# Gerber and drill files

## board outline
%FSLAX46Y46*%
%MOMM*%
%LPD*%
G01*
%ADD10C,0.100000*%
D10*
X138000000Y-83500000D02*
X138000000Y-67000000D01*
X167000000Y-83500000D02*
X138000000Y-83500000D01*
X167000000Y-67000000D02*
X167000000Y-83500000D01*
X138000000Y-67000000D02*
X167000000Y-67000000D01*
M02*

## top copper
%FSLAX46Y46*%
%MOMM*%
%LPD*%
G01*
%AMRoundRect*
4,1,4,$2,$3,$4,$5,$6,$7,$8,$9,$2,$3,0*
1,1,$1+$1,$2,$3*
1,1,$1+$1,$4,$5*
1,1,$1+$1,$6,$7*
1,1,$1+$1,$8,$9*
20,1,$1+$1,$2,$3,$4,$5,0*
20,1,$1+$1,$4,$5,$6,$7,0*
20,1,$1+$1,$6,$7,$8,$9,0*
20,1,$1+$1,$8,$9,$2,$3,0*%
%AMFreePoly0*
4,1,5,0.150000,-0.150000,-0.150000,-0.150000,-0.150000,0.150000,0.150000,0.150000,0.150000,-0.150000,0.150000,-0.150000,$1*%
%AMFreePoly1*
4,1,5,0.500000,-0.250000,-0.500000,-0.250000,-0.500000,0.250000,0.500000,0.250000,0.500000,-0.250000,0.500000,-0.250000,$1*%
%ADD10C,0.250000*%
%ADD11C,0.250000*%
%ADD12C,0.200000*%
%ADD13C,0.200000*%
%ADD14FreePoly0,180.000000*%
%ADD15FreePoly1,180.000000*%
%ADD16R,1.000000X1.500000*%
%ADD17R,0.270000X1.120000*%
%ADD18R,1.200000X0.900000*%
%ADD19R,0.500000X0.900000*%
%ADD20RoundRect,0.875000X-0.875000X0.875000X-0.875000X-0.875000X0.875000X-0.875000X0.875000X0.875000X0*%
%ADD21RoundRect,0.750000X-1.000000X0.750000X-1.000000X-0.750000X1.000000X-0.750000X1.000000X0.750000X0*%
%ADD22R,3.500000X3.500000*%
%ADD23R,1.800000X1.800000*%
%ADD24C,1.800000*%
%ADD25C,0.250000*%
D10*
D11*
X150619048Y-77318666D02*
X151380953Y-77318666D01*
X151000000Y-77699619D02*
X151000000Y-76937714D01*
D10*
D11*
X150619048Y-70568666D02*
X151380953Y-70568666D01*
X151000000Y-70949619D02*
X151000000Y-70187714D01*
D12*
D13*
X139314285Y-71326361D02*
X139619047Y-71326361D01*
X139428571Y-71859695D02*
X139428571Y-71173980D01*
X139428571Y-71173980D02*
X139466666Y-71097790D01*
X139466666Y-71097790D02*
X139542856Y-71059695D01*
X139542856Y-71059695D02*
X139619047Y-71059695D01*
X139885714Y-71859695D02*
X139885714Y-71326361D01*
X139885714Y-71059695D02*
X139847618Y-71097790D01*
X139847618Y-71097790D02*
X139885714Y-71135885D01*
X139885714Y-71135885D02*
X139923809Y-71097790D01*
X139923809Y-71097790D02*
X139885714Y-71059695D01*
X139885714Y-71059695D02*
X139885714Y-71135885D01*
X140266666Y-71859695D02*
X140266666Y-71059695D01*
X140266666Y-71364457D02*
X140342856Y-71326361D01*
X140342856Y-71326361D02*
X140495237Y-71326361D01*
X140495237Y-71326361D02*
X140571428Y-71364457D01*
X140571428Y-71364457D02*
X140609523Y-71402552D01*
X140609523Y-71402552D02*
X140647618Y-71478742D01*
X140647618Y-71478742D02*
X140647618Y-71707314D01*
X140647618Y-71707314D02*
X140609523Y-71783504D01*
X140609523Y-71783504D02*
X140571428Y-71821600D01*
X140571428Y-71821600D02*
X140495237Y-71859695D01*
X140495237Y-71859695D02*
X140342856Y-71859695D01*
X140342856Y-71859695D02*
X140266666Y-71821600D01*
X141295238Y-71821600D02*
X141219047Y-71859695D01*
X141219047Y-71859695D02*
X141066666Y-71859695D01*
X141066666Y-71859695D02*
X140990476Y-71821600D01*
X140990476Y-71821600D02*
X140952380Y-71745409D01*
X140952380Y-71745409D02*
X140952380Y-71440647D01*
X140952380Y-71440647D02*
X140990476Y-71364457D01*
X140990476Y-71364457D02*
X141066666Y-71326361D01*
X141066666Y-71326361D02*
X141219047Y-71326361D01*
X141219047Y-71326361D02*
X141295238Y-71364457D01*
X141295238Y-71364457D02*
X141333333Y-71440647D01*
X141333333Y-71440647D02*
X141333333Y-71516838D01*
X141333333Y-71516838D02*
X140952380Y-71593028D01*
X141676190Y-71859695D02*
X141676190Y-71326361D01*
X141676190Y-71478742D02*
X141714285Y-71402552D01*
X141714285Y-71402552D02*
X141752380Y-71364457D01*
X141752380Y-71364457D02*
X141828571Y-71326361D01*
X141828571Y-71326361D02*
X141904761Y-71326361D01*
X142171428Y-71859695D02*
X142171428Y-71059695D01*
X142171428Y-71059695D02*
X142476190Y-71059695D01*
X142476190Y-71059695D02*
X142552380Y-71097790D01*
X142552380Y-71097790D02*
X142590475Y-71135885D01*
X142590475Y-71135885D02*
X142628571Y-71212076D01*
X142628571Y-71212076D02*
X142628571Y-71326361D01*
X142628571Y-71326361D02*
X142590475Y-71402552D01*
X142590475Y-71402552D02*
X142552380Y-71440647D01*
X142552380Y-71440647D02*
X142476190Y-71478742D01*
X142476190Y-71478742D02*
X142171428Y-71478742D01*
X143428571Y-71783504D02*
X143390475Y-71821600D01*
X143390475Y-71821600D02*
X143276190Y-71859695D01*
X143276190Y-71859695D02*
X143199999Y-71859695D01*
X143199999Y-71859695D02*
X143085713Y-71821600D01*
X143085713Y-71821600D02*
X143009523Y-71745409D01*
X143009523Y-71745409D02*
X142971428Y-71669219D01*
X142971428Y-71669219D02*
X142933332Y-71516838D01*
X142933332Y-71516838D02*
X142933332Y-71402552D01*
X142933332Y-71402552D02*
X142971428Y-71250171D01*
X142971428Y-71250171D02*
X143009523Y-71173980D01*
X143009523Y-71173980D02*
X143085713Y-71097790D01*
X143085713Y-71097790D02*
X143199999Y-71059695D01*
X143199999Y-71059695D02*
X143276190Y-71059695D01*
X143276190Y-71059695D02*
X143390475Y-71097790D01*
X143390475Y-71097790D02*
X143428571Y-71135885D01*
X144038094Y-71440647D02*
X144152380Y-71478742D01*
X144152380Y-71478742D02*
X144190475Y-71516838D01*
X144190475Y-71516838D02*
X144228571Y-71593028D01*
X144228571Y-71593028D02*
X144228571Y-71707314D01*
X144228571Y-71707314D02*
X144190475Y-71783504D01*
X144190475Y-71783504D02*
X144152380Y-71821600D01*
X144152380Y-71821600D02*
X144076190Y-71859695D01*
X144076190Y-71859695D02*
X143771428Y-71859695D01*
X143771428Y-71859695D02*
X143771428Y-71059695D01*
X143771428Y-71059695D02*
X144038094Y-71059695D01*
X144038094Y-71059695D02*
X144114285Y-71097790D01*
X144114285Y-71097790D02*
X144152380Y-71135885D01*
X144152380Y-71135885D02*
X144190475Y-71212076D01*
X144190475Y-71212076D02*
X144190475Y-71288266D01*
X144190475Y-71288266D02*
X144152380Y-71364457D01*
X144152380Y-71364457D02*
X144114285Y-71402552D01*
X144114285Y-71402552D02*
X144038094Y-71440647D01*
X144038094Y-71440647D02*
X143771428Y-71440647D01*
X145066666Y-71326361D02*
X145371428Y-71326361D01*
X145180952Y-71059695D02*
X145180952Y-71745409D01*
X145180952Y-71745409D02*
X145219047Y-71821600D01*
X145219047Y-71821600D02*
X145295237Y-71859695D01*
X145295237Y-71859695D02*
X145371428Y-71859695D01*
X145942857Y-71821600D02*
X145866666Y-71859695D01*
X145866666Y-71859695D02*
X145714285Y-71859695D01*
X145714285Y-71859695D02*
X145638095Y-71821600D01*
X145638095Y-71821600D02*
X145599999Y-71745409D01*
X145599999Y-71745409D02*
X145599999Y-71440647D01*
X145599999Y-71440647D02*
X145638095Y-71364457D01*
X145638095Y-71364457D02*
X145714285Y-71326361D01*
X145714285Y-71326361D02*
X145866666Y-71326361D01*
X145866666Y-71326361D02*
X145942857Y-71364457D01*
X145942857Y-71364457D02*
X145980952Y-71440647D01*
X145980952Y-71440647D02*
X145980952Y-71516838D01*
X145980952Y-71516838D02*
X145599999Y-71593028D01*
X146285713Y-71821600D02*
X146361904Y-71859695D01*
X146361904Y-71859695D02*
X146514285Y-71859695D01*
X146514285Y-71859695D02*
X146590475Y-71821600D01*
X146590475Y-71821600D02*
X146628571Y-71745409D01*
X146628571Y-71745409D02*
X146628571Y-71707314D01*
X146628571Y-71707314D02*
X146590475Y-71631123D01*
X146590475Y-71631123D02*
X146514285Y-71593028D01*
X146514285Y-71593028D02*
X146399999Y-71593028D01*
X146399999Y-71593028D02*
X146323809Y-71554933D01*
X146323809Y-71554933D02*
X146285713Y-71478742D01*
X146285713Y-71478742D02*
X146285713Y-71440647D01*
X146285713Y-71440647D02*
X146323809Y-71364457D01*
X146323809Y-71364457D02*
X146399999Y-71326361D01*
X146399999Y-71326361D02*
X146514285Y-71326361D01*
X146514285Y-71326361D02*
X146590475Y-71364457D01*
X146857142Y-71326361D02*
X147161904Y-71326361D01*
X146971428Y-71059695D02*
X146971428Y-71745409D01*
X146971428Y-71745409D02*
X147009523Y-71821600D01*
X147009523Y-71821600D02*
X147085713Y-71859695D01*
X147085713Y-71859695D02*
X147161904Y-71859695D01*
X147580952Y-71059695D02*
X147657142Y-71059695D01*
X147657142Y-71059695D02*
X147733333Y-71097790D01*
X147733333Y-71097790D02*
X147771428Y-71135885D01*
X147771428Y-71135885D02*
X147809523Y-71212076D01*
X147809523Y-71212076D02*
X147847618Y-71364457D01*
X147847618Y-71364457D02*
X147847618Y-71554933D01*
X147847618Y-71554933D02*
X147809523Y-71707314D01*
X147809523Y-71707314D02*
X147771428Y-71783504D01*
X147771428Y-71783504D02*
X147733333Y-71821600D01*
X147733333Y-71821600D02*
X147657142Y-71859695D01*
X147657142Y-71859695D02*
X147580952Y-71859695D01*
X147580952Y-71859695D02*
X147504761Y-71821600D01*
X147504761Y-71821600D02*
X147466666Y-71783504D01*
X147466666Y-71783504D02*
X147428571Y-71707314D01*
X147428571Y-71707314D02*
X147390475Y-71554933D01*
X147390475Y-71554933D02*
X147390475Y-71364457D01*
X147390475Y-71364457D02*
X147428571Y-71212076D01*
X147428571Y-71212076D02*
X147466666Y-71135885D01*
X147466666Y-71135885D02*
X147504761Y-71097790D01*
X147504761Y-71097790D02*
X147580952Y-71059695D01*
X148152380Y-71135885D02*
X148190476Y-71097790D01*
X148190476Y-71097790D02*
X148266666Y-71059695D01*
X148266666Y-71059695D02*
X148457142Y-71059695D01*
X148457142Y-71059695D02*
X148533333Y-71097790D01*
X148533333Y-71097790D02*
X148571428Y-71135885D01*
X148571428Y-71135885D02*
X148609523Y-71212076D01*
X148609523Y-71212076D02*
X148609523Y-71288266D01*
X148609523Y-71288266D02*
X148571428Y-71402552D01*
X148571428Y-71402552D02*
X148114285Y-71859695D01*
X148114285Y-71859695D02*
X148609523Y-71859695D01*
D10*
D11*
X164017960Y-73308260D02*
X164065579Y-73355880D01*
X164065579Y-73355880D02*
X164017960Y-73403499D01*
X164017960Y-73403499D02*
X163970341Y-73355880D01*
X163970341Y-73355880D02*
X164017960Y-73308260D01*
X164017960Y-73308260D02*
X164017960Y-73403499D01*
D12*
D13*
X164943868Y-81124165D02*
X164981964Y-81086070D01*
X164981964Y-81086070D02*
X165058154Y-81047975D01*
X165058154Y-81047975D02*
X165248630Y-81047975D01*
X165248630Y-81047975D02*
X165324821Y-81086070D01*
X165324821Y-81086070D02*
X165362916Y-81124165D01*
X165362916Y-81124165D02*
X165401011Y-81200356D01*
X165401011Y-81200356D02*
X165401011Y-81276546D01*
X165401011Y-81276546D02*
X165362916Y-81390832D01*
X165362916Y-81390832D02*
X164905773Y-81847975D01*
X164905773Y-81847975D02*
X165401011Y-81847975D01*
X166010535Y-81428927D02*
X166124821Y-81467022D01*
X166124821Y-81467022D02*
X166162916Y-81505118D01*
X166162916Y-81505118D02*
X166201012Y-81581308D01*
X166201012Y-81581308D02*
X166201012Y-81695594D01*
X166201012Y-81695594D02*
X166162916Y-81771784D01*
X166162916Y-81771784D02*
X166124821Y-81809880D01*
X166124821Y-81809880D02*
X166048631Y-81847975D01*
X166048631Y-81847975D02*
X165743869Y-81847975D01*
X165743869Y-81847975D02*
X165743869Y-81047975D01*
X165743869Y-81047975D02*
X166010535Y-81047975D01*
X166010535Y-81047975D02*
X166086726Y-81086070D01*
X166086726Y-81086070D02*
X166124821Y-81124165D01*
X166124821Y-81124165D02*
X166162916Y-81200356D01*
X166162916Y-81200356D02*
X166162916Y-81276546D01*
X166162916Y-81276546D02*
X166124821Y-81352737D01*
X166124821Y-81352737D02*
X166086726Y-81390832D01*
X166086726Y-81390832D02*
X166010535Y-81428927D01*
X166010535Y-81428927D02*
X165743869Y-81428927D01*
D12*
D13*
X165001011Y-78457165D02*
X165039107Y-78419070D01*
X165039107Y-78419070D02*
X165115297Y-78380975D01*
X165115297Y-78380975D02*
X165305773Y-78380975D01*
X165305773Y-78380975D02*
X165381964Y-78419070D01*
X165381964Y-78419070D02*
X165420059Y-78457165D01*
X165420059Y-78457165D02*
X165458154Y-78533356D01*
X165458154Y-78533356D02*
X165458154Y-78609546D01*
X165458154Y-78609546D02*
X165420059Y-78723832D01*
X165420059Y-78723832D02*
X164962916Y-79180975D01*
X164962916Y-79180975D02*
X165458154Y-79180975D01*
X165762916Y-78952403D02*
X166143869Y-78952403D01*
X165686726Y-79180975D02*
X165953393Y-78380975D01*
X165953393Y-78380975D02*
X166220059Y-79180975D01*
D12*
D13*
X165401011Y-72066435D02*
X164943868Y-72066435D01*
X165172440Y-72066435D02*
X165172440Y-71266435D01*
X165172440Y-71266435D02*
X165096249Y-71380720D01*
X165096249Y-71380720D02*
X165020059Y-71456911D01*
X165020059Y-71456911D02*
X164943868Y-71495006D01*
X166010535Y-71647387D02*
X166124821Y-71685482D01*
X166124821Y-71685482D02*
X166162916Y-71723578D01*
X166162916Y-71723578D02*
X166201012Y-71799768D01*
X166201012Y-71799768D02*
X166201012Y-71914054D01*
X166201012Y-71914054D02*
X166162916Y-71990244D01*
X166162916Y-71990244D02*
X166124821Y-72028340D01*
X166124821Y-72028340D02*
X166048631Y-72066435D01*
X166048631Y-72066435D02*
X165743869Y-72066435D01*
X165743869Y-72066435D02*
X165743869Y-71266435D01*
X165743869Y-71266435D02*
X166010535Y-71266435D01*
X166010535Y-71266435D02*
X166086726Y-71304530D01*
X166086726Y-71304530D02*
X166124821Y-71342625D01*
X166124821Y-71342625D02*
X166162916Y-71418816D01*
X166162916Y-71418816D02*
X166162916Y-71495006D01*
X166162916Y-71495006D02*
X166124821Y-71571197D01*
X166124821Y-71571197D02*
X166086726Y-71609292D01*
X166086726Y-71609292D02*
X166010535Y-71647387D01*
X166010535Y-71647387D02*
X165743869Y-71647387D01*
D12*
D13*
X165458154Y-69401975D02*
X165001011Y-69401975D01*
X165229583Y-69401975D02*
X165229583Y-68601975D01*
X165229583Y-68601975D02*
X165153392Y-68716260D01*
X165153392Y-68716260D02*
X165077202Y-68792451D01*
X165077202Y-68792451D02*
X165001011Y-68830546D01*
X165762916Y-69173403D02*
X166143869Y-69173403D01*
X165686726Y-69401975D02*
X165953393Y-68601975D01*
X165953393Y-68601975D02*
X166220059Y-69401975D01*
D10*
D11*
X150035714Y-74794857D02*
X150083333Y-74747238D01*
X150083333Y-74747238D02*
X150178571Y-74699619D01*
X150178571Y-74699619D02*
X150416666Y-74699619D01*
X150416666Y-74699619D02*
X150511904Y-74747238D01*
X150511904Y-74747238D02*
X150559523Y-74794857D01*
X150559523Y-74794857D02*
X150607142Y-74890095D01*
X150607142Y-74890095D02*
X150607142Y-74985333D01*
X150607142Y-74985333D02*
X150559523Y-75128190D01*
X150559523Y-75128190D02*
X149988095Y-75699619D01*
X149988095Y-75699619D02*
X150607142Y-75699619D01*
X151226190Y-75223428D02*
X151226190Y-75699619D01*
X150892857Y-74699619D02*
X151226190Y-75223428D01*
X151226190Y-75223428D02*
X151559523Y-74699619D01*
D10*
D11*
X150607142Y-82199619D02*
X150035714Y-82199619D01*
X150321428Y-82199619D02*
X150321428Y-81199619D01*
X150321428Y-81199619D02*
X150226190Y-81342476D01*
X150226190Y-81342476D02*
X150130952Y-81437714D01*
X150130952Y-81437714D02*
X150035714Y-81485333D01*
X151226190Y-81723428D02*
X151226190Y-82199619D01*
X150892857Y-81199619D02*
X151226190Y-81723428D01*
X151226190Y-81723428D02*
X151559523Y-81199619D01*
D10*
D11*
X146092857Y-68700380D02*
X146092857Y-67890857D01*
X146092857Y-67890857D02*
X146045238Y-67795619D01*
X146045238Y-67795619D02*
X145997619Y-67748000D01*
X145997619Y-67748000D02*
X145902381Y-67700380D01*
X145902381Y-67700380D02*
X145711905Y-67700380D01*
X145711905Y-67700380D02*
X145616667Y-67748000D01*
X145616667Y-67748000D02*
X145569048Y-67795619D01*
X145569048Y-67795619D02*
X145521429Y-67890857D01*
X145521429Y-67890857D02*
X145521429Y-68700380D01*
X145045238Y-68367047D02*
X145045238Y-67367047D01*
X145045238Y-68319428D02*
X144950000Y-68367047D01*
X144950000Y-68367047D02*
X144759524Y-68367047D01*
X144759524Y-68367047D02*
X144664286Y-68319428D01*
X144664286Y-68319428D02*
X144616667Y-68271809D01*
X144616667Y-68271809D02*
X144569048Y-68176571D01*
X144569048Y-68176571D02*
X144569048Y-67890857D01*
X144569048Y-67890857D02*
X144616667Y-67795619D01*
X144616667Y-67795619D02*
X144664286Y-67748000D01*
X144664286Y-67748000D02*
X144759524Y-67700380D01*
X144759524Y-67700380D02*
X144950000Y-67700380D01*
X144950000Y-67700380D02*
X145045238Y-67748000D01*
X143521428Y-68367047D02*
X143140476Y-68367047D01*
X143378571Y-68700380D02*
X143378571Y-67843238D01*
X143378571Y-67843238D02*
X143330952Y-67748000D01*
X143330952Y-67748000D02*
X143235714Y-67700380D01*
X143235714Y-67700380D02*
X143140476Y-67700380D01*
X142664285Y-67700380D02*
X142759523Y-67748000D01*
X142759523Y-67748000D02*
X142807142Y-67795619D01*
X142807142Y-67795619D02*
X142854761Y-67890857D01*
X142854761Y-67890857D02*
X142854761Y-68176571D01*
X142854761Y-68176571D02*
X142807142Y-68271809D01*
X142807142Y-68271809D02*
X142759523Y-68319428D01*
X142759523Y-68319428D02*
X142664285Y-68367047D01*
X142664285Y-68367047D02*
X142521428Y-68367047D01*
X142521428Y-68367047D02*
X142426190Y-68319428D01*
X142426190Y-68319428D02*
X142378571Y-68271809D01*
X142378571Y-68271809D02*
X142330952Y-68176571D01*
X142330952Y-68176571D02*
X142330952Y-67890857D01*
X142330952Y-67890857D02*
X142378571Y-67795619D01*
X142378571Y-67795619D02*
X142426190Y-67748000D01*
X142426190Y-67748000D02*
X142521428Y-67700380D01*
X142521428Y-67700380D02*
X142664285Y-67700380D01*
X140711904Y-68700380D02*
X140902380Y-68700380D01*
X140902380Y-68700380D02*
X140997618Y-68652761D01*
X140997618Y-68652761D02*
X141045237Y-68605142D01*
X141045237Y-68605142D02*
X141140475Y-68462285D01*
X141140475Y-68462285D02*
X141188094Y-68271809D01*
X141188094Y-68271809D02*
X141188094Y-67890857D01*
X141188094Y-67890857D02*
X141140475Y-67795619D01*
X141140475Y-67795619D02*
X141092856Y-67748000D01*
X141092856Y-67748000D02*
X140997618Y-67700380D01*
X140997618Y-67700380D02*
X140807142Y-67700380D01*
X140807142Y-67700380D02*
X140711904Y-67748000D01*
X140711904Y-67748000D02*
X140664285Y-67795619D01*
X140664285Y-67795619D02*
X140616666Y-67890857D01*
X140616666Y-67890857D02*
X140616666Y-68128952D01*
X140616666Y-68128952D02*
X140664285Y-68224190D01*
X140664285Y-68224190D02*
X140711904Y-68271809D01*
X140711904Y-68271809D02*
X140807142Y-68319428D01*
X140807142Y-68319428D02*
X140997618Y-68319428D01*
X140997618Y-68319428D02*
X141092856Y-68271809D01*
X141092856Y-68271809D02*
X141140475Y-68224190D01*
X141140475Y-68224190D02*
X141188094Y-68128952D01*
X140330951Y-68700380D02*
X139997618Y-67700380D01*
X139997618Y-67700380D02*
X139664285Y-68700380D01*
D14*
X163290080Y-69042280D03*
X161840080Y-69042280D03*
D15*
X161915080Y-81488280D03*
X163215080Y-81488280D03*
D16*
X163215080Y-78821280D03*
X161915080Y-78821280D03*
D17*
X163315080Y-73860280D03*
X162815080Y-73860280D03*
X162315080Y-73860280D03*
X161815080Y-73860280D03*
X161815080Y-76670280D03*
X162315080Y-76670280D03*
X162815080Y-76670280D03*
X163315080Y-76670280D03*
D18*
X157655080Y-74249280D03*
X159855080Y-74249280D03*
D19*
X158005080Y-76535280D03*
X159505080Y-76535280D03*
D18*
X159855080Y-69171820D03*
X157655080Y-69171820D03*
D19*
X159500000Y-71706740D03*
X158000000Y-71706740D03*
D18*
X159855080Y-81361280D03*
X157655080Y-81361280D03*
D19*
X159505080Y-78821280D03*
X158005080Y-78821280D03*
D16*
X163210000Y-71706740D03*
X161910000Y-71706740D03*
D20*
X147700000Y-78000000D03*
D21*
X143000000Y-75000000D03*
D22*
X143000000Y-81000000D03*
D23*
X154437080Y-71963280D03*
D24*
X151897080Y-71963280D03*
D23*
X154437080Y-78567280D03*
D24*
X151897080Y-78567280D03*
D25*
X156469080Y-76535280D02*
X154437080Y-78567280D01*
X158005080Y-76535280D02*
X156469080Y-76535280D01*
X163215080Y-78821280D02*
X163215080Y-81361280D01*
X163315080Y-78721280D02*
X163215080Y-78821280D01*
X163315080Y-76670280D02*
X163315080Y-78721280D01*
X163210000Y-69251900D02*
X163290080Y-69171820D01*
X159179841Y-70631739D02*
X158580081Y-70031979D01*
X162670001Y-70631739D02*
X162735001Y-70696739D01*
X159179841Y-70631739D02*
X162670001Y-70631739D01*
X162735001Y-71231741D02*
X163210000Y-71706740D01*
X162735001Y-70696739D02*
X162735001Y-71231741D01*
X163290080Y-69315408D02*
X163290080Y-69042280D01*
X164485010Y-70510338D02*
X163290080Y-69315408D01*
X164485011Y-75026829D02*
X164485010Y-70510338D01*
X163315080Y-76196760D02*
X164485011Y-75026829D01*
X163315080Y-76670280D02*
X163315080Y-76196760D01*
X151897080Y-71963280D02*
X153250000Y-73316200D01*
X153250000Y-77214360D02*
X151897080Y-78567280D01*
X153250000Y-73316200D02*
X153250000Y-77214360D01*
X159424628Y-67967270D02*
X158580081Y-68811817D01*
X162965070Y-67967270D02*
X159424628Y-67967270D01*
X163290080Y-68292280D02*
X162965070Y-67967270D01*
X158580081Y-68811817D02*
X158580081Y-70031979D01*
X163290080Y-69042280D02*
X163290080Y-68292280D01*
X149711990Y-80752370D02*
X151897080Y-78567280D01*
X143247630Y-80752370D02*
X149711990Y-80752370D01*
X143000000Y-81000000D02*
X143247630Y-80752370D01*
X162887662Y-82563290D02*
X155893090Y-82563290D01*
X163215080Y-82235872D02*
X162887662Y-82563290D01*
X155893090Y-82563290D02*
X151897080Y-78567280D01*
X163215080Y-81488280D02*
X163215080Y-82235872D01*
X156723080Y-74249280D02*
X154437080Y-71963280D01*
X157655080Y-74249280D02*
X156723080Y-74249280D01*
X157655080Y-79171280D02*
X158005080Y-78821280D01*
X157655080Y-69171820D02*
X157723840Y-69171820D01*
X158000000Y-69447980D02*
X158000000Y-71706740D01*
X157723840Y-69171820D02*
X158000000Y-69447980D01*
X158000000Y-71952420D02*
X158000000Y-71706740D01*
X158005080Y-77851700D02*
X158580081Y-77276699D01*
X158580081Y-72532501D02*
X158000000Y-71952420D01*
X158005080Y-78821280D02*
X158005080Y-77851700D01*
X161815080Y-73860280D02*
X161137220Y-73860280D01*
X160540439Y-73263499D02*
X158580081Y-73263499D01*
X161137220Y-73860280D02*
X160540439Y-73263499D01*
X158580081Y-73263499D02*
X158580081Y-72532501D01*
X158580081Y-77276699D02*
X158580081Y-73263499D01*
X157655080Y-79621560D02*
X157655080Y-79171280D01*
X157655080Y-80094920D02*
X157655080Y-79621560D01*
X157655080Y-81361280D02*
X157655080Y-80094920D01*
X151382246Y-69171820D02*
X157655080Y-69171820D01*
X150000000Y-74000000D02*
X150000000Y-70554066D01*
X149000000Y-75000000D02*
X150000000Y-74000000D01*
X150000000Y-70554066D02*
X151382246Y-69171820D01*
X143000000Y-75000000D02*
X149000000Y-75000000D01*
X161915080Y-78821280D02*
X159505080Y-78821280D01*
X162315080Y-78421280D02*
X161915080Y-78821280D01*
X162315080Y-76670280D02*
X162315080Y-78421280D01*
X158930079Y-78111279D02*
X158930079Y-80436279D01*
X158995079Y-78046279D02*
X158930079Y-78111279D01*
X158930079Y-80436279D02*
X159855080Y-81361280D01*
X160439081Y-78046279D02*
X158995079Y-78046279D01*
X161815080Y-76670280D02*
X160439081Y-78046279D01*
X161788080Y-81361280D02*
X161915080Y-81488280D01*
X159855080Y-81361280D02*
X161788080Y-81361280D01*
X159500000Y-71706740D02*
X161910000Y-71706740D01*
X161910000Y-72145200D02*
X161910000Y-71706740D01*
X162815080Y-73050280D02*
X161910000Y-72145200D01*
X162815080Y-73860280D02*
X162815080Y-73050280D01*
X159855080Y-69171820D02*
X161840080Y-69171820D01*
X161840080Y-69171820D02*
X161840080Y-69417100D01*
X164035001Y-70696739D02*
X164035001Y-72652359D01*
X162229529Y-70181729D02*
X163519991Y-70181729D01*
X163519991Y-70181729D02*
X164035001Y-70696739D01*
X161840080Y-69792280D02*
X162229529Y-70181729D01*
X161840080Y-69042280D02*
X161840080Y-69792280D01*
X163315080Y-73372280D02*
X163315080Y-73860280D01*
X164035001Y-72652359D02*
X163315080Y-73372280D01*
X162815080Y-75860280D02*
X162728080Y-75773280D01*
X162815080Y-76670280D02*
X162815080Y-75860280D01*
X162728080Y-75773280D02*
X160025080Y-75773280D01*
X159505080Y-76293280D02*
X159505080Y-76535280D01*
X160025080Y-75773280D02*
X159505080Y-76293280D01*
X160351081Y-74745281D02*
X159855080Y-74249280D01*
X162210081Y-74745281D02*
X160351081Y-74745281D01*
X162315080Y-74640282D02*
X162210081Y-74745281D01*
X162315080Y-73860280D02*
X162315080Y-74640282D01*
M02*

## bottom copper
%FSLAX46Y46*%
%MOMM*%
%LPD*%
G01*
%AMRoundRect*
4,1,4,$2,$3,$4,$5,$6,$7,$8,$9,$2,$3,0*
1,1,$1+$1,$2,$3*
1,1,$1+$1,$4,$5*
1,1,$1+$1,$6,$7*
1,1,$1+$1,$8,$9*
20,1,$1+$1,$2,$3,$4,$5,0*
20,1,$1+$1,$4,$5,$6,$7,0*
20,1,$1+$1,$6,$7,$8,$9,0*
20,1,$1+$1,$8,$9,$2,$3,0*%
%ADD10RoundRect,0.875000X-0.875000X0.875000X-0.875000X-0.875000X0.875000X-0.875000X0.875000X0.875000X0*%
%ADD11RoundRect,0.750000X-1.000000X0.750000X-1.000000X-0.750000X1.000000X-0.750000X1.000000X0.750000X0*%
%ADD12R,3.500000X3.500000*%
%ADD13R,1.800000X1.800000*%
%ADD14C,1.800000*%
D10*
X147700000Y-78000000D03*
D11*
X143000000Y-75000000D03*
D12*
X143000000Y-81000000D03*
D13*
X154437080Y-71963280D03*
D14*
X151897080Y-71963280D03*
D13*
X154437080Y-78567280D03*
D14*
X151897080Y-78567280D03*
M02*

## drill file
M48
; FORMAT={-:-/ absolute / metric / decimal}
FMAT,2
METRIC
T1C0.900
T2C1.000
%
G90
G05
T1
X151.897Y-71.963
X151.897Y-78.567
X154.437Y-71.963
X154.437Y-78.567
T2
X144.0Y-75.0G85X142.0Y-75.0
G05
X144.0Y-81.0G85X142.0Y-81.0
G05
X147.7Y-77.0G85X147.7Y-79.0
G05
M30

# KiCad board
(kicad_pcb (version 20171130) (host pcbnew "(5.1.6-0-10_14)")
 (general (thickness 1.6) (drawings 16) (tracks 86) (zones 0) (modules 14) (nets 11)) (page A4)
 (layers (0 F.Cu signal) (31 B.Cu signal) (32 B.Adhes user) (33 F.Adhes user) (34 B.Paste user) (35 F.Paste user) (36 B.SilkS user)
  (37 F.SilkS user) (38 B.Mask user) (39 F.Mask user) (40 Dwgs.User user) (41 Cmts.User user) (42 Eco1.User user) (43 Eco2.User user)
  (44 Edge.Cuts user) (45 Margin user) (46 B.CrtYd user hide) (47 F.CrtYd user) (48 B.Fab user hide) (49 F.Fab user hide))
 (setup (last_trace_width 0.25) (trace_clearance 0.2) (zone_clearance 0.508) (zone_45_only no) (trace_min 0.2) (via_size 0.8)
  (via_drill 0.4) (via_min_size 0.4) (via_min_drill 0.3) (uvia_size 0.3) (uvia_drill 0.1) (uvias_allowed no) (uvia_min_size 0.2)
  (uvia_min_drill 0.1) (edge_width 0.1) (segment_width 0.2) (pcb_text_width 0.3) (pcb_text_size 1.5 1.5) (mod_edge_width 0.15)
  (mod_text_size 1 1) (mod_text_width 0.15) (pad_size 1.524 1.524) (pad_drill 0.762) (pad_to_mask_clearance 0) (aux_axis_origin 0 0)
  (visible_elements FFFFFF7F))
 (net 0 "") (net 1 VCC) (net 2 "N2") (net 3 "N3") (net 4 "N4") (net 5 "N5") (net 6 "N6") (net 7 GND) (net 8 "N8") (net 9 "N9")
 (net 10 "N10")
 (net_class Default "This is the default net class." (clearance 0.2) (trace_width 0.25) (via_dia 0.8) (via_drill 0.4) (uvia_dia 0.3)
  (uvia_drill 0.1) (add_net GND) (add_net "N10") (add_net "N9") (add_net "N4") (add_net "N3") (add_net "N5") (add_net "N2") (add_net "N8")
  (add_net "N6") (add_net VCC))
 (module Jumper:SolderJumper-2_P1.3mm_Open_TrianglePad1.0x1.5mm (layer F.Cu) (at 162.56508 69.04228 180)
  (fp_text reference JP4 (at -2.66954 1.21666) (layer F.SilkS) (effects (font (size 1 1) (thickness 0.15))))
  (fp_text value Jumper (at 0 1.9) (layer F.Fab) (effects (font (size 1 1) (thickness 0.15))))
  (pad 1 smd custom (at -0.725 0 180) (size 0.3 0.3) (layers F.Cu F.Mask) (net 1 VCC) (zone_connect 2)
   (options (clearance outline) (anchor rect)) (primitives))
  (pad 2 smd custom (at 0.725 0 180) (size 0.3 0.3) (layers F.Cu F.Mask) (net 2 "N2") (zone_connect 2)
   (options (clearance outline) (anchor rect)) (primitives)))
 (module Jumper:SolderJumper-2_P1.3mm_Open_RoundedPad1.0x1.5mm (layer F.Cu) (at 162.56508 81.48828 180)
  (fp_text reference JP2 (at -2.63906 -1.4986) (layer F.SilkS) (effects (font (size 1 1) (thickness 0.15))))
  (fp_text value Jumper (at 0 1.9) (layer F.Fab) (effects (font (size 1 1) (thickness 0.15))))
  (pad 2 smd custom (at 0.65 0 180) (size 1 0.5) (layers F.Cu F.Mask) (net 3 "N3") (zone_connect 2)
   (options (clearance outline) (anchor rect)) (primitives))
  (pad 1 smd custom (at -0.65 0 180) (size 1 0.5) (layers F.Cu F.Mask) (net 1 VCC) (zone_connect 2)
   (options (clearance outline) (anchor rect)) (primitives)))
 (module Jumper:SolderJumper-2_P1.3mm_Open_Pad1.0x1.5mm (layer F.Cu) (at 162.56508 78.82128 180)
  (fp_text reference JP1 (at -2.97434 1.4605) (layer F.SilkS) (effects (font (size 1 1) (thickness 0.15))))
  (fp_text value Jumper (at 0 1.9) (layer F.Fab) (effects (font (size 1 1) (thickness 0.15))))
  (pad 1 smd rect (at -0.65 0 180) (size 1 1.5) (layers F.Cu F.Mask) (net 1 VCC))
  (pad 2 smd rect (at 0.65 0 180) (size 1 1.5) (layers F.Cu F.Mask) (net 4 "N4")))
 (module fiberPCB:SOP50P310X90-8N (layer F.Cu) (at 162.56508 75.26528 270)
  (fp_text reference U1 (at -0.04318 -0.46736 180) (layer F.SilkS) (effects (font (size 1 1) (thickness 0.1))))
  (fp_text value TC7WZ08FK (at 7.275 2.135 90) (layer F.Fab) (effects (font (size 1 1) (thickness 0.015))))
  (pad 1 smd rect (at -1.405 -0.75 270) (size 1.12 0.27) (layers F.Cu F.Paste F.Mask) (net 2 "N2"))
  (pad 2 smd rect (at -1.405 -0.25 270) (size 1.12 0.27) (layers F.Cu F.Paste F.Mask) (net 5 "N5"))
  (pad 3 smd rect (at -1.405 0.25 270) (size 1.12 0.27) (layers F.Cu F.Paste F.Mask) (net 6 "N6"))
  (pad 4 smd rect (at -1.405 0.75 270) (size 1.12 0.27) (layers F.Cu F.Paste F.Mask) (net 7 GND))
  (pad 5 smd rect (at 1.405 0.75 270) (size 1.12 0.27) (layers F.Cu F.Paste F.Mask) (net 3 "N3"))
  (pad 6 smd rect (at 1.405 0.25 270) (size 1.12 0.27) (layers F.Cu F.Paste F.Mask) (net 4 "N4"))
  (pad 7 smd rect (at 1.405 -0.25 270) (size 1.12 0.27) (layers F.Cu F.Paste F.Mask) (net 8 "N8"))
  (pad 8 smd rect (at 1.405 -0.75 270) (size 1.12 0.27) (layers F.Cu F.Paste F.Mask) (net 1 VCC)))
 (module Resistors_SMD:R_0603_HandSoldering (layer F.Cu) (at 158.75508 74.24928)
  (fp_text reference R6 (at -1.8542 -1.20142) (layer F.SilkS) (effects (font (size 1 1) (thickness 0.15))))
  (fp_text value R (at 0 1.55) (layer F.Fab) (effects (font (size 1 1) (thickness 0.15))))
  (pad 1 smd rect (at -1.1 0) (size 1.2 0.9) (layers F.Cu F.Paste F.Mask) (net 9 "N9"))
  (pad 2 smd rect (at 1.1 0) (size 1.2 0.9) (layers F.Cu F.Paste F.Mask) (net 6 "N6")))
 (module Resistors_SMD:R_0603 (layer F.Cu) (at 158.75508 76.53528)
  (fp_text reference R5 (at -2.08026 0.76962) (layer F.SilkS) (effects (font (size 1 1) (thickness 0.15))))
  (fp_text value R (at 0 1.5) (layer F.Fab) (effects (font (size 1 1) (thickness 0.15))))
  (pad 1 smd rect (at -0.75 0) (size 0.5 0.9) (layers F.Cu F.Paste F.Mask) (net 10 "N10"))
  (pad 2 smd rect (at 0.75 0) (size 0.5 0.9) (layers F.Cu F.Paste F.Mask) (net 8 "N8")))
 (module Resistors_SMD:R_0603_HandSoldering (layer F.Cu) (at 158.75508 69.17182 180)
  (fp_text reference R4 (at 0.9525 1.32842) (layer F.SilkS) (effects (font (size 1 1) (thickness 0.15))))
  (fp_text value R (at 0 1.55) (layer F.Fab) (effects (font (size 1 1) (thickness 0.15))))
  (pad 1 smd rect (at -1.1 0 180) (size 1.2 0.9) (layers F.Cu F.Paste F.Mask) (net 2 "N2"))
  (pad 2 smd rect (at 1.1 0 180) (size 1.2 0.9) (layers F.Cu F.Paste F.Mask) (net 7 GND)))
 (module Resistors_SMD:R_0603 (layer F.Cu) (at 158.75 71.70674 180)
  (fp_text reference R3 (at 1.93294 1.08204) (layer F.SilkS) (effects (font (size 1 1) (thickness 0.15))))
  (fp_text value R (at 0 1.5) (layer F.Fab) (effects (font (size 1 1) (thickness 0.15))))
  (pad 1 smd rect (at -0.75 0 180) (size 0.5 0.9) (layers F.Cu F.Paste F.Mask) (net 5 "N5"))
  (pad 2 smd rect (at 0.75 0 180) (size 0.5 0.9) (layers F.Cu F.Paste F.Mask) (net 7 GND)))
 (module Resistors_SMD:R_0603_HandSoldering (layer F.Cu) (at 158.75508 81.36128 180)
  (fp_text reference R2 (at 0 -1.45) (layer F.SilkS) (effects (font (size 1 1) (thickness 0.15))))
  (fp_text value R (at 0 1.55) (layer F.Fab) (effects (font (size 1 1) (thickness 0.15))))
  (pad 1 smd rect (at -1.1 0 180) (size 1.2 0.9) (layers F.Cu F.Paste F.Mask) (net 3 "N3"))
  (pad 2 smd rect (at 1.1 0 180) (size 1.2 0.9) (layers F.Cu F.Paste F.Mask) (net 7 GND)))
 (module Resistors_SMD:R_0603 (layer F.Cu) (at 158.75508 78.82128 180)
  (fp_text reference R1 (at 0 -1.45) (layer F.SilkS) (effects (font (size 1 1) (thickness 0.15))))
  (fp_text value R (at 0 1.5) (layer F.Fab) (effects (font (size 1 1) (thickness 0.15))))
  (pad 1 smd rect (at -0.75 0 180) (size 0.5 0.9) (layers F.Cu F.Paste F.Mask) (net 4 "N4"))
  (pad 2 smd rect (at 0.75 0 180) (size 0.5 0.9) (layers F.Cu F.Paste F.Mask) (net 7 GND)))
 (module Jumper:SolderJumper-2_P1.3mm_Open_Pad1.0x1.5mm (layer F.Cu) (at 162.56 71.70674 180)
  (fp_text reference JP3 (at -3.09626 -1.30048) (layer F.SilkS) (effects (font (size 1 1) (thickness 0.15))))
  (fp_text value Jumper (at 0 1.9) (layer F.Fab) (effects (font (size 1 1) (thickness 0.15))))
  (pad 1 smd rect (at -0.65 0 180) (size 1 1.5) (layers F.Cu F.Mask) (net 1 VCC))
  (pad 2 smd rect (at 0.65 0 180) (size 1 1.5) (layers F.Cu F.Mask) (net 5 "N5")))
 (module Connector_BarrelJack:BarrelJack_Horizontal (layer B.Cu) (at 143 81 270)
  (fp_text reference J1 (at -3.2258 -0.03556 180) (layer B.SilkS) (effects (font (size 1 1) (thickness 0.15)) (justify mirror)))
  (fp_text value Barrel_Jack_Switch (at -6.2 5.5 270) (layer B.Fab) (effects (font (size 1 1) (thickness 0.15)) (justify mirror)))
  (pad 3 thru_hole roundrect (at -3 -4.7 270) (size 3.5 3.5) (drill oval 3 1) (layers *.Cu *.Mask) (roundrect_rratio 0.25))
  (pad 2 thru_hole roundrect (at -6 0 270) (size 3 3.5) (drill oval 1 3) (layers *.Cu *.Mask) (roundrect_rratio 0.25) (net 7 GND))
  (pad 1 thru_hole rect (at 0 0 270) (size 3.5 3.5) (drill oval 1 3) (layers *.Cu *.Mask) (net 1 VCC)))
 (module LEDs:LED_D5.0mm (layer F.Cu) (at 154.43708 71.96328 180)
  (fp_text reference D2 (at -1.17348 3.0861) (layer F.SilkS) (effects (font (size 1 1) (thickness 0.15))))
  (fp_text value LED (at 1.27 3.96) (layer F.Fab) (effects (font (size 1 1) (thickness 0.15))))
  (pad 1 thru_hole rect (at 0 0 180) (size 1.8 1.8) (drill 0.9) (layers *.Cu *.Mask) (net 9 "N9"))
  (pad 2 thru_hole circle (at 2.54 0 180) (size 1.8 1.8) (drill 0.9) (layers *.Cu *.Mask) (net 1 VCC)))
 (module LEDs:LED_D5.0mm (layer F.Cu) (at 154.43708 78.56728 180)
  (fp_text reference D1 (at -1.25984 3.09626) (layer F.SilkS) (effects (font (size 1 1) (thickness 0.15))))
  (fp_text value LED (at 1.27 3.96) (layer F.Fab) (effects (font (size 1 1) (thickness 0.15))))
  (pad 1 thru_hole rect (at 0 0 180) (size 1.8 1.8) (drill 0.9) (layers *.Cu *.Mask) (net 10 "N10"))
  (pad 2 thru_hole circle (at 2.54 0 180) (size 1.8 1.8) (drill 0.9) (layers *.Cu *.Mask) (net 1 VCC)))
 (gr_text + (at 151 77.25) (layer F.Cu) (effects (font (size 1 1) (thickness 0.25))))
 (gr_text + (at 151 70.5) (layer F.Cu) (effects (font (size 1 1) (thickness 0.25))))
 (gr_line (start 138 83.5) (end 138 67) (layer Edge.Cuts) (width 0.1))
 (gr_line (start 167 83.5) (end 138 83.5) (layer Edge.Cuts) (width 0.1))
 (gr_line (start 167 67) (end 167 83.5) (layer Edge.Cuts) (width 0.1))
 (gr_line (start 138 67) (end 167 67) (layer Edge.Cuts) (width 0.1))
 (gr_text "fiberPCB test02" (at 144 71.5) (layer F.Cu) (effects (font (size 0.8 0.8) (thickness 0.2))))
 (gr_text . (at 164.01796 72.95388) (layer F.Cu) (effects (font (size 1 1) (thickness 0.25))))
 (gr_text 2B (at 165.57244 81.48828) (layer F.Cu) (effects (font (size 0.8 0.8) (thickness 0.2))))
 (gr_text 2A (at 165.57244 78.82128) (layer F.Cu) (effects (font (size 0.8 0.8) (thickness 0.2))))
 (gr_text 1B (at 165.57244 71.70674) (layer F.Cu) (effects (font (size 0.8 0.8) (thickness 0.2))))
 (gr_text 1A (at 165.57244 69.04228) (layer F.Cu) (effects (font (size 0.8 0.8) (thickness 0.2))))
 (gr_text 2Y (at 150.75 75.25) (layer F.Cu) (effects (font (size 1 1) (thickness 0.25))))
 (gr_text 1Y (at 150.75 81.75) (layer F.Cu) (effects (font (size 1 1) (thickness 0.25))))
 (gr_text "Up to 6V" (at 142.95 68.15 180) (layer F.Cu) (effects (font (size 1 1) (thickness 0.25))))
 (segment (start 156.46908 76.53528) (end 154.43708 78.56728) (width 0.25) (layer F.Cu) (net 10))
 (segment (start 158.00508 76.53528) (end 156.46908 76.53528) (width 0.25) (layer F.Cu) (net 10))
 (segment (start 163.21508 78.82128) (end 163.21508 81.36128) (width 0.25) (layer F.Cu) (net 1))
 (segment (start 163.31508 78.72128) (end 163.21508 78.82128) (width 0.25) (layer F.Cu) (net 1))
 (segment (start 163.31508 76.67028) (end 163.31508 78.72128) (width 0.25) (layer F.Cu) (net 1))
 (segment (start 163.21 69.2519) (end 163.29008 69.17182) (width 0.25) (layer F.Cu) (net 1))
 (segment (start 159.179841 70.631739) (end 158.580081 70.031979) (width 0.25) (layer F.Cu) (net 1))
 (segment (start 162.670001 70.631739) (end 162.735001 70.696739) (width 0.25) (layer F.Cu) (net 1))
 (segment (start 159.179841 70.631739) (end 162.670001 70.631739) (width 0.25) (layer F.Cu) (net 1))
 (segment (start 162.735001 71.231741) (end 163.21 71.70674) (width 0.25) (layer F.Cu) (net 1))
 (segment (start 162.735001 70.696739) (end 162.735001 71.231741) (width 0.25) (layer F.Cu) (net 1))
 (segment (start 163.29008 69.315408) (end 163.29008 69.04228) (width 0.25) (layer F.Cu) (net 1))
 (segment (start 164.48501 70.510338) (end 163.29008 69.315408) (width 0.25) (layer F.Cu) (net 1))
 (segment (start 164.485011 75.026829) (end 164.48501 70.510338) (width 0.25) (layer F.Cu) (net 1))
 (segment (start 163.31508 76.19676) (end 164.485011 75.026829) (width 0.25) (layer F.Cu) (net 1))
 (segment (start 163.31508 76.67028) (end 163.31508 76.19676) (width 0.25) (layer F.Cu) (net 1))
 (segment (start 151.89708 71.96328) (end 153.25 73.3162) (width 0.25) (layer F.Cu) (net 1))
 (segment (start 153.25 77.21436) (end 151.89708 78.56728) (width 0.25) (layer F.Cu) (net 1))
 (segment (start 153.25 73.3162) (end 153.25 77.21436) (width 0.25) (layer F.Cu) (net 1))
 (segment (start 159.424628 67.96727) (end 158.580081 68.811817) (width 0.25) (layer F.Cu) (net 1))
 (segment (start 162.96507 67.96727) (end 159.424628 67.96727) (width 0.25) (layer F.Cu) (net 1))
 (segment (start 163.29008 68.29228) (end 162.96507 67.96727) (width 0.25) (layer F.Cu) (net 1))
 (segment (start 158.580081 68.811817) (end 158.580081 70.031979) (width 0.25) (layer F.Cu) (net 1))
 (segment (start 163.29008 69.04228) (end 163.29008 68.29228) (width 0.25) (layer F.Cu) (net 1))
 (segment (start 149.71199 80.75237) (end 151.89708 78.56728) (width 0.25) (layer F.Cu) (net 1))
 (segment (start 143.24763 80.75237) (end 149.71199 80.75237) (width 0.25) (layer F.Cu) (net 1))
 (segment (start 143 81) (end 143.24763 80.75237) (width 0.25) (layer F.Cu) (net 1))
 (segment (start 162.887662 82.56329) (end 155.89309 82.56329) (width 0.25) (layer F.Cu) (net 1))
 (segment (start 163.21508 82.235872) (end 162.887662 82.56329) (width 0.25) (layer F.Cu) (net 1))
 (segment (start 155.89309 82.56329) (end 151.89708 78.56728) (width 0.25) (layer F.Cu) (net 1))
 (segment (start 163.21508 81.48828) (end 163.21508 82.235872) (width 0.25) (layer F.Cu) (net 1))
 (segment (start 156.72308 74.24928) (end 154.43708 71.96328) (width 0.25) (layer F.Cu) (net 9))
 (segment (start 157.65508 74.24928) (end 156.72308 74.24928) (width 0.25) (layer F.Cu) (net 9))
 (segment (start 157.65508 79.17128) (end 158.00508 78.82128) (width 0.25) (layer F.Cu) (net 7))
 (segment (start 157.65508 69.17182) (end 157.72384 69.17182) (width 0.25) (layer F.Cu) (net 7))
 (segment (start 158 69.44798) (end 158 71.70674) (width 0.25) (layer F.Cu) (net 7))
 (segment (start 157.72384 69.17182) (end 158 69.44798) (width 0.25) (layer F.Cu) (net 7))
 (segment (start 158 71.95242) (end 158 71.70674) (width 0.25) (layer F.Cu) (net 7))
 (segment (start 158.00508 77.8517) (end 158.580081 77.276699) (width 0.25) (layer F.Cu) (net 7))
 (segment (start 158.580081 72.532501) (end 158 71.95242) (width 0.25) (layer F.Cu) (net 7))
 (segment (start 158.00508 78.82128) (end 158.00508 77.8517) (width 0.25) (layer F.Cu) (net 7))
 (segment (start 161.81508 73.86028) (end 161.13722 73.86028) (width 0.25) (layer F.Cu) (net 7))
 (segment (start 160.540439 73.263499) (end 158.580081 73.263499) (width 0.25) (layer F.Cu) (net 7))
 (segment (start 161.13722 73.86028) (end 160.540439 73.263499) (width 0.25) (layer F.Cu) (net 7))
 (segment (start 158.580081 73.263499) (end 158.580081 72.532501) (width 0.25) (layer F.Cu) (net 7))
 (segment (start 158.580081 77.276699) (end 158.580081 73.263499) (width 0.25) (layer F.Cu) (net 7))
 (segment (start 157.65508 79.62156) (end 157.65508 79.17128) (width 0.25) (layer F.Cu) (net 7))
 (segment (start 157.65508 80.09492) (end 157.65508 79.62156) (width 0.25) (layer F.Cu) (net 7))
 (segment (start 157.65508 81.36128) (end 157.65508 80.09492) (width 0.25) (layer F.Cu) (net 7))
 (segment (start 151.382246 69.17182) (end 157.65508 69.17182) (width 0.25) (layer F.Cu) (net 7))
 (segment (start 150 74) (end 150 70.554066) (width 0.25) (layer F.Cu) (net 7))
 (segment (start 149 75) (end 150 74) (width 0.25) (layer F.Cu) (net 7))
 (segment (start 150 70.554066) (end 151.382246 69.17182) (width 0.25) (layer F.Cu) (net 7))
 (segment (start 143 75) (end 149 75) (width 0.25) (layer F.Cu) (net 7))
 (segment (start 161.91508 78.82128) (end 159.50508 78.82128) (width 0.25) (layer F.Cu) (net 4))
 (segment (start 162.31508 78.42128) (end 161.91508 78.82128) (width 0.25) (layer F.Cu) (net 4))
 (segment (start 162.31508 76.67028) (end 162.31508 78.42128) (width 0.25) (layer F.Cu) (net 4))
 (segment (start 158.930079 78.111279) (end 158.930079 80.436279) (width 0.25) (layer F.Cu) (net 3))
 (segment (start 158.995079 78.046279) (end 158.930079 78.111279) (width 0.25) (layer F.Cu) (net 3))
 (segment (start 158.930079 80.436279) (end 159.85508 81.36128) (width 0.25) (layer F.Cu) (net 3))
 (segment (start 160.439081 78.046279) (end 158.995079 78.046279) (width 0.25) (layer F.Cu) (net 3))
 (segment (start 161.81508 76.67028) (end 160.439081 78.046279) (width 0.25) (layer F.Cu) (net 3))
 (segment (start 161.78808 81.36128) (end 161.91508 81.48828) (width 0.25) (layer F.Cu) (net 3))
 (segment (start 159.85508 81.36128) (end 161.78808 81.36128) (width 0.25) (layer F.Cu) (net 3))
 (segment (start 159.5 71.70674) (end 161.91 71.70674) (width 0.25) (layer F.Cu) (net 5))
 (segment (start 161.91 72.1452) (end 161.91 71.70674) (width 0.25) (layer F.Cu) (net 5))
 (segment (start 162.81508 73.05028) (end 161.91 72.1452) (width 0.25) (layer F.Cu) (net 5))
 (segment (start 162.81508 73.86028) (end 162.81508 73.05028) (width 0.25) (layer F.Cu) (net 5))
 (segment (start 159.85508 69.17182) (end 161.84008 69.17182) (width 0.25) (layer F.Cu) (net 2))
 (segment (start 161.84008 69.17182) (end 161.84008 69.4171) (width 0.25) (layer F.Cu) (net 2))
 (segment (start 164.035001 70.696739) (end 164.035001 72.652359) (width 0.25) (layer F.Cu) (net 2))
 (segment (start 162.229529 70.181729) (end 163.519991 70.181729) (width 0.25) (layer F.Cu) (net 2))
 (segment (start 163.519991 70.181729) (end 164.035001 70.696739) (width 0.25) (layer F.Cu) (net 2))
 (segment (start 161.84008 69.79228) (end 162.229529 70.181729) (width 0.25) (layer F.Cu) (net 2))
 (segment (start 161.84008 69.04228) (end 161.84008 69.79228) (width 0.25) (layer F.Cu) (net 2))
 (segment (start 163.31508 73.37228) (end 163.31508 73.86028) (width 0.25) (layer F.Cu) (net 2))
 (segment (start 164.035001 72.652359) (end 163.31508 73.37228) (width 0.25) (layer F.Cu) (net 2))
 (segment (start 162.81508 75.86028) (end 162.72808 75.77328) (width 0.25) (layer F.Cu) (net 8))
 (segment (start 162.81508 76.67028) (end 162.81508 75.86028) (width 0.25) (layer F.Cu) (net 8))
 (segment (start 162.72808 75.77328) (end 160.02508 75.77328) (width 0.25) (layer F.Cu) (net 8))
 (segment (start 159.50508 76.29328) (end 159.50508 76.53528) (width 0.25) (layer F.Cu) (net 8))
 (segment (start 160.02508 75.77328) (end 159.50508 76.29328) (width 0.25) (layer F.Cu) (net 8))
 (segment (start 160.351081 74.745281) (end 159.85508 74.24928) (width 0.25) (layer F.Cu) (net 6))
 (segment (start 162.210081 74.745281) (end 160.351081 74.745281) (width 0.25) (layer F.Cu) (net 6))
 (segment (start 162.31508 74.640282) (end 162.210081 74.745281) (width 0.25) (layer F.Cu) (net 6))
 (segment (start 162.31508 73.86028) (end 162.31508 74.640282) (width 0.25) (layer F.Cu) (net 6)))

